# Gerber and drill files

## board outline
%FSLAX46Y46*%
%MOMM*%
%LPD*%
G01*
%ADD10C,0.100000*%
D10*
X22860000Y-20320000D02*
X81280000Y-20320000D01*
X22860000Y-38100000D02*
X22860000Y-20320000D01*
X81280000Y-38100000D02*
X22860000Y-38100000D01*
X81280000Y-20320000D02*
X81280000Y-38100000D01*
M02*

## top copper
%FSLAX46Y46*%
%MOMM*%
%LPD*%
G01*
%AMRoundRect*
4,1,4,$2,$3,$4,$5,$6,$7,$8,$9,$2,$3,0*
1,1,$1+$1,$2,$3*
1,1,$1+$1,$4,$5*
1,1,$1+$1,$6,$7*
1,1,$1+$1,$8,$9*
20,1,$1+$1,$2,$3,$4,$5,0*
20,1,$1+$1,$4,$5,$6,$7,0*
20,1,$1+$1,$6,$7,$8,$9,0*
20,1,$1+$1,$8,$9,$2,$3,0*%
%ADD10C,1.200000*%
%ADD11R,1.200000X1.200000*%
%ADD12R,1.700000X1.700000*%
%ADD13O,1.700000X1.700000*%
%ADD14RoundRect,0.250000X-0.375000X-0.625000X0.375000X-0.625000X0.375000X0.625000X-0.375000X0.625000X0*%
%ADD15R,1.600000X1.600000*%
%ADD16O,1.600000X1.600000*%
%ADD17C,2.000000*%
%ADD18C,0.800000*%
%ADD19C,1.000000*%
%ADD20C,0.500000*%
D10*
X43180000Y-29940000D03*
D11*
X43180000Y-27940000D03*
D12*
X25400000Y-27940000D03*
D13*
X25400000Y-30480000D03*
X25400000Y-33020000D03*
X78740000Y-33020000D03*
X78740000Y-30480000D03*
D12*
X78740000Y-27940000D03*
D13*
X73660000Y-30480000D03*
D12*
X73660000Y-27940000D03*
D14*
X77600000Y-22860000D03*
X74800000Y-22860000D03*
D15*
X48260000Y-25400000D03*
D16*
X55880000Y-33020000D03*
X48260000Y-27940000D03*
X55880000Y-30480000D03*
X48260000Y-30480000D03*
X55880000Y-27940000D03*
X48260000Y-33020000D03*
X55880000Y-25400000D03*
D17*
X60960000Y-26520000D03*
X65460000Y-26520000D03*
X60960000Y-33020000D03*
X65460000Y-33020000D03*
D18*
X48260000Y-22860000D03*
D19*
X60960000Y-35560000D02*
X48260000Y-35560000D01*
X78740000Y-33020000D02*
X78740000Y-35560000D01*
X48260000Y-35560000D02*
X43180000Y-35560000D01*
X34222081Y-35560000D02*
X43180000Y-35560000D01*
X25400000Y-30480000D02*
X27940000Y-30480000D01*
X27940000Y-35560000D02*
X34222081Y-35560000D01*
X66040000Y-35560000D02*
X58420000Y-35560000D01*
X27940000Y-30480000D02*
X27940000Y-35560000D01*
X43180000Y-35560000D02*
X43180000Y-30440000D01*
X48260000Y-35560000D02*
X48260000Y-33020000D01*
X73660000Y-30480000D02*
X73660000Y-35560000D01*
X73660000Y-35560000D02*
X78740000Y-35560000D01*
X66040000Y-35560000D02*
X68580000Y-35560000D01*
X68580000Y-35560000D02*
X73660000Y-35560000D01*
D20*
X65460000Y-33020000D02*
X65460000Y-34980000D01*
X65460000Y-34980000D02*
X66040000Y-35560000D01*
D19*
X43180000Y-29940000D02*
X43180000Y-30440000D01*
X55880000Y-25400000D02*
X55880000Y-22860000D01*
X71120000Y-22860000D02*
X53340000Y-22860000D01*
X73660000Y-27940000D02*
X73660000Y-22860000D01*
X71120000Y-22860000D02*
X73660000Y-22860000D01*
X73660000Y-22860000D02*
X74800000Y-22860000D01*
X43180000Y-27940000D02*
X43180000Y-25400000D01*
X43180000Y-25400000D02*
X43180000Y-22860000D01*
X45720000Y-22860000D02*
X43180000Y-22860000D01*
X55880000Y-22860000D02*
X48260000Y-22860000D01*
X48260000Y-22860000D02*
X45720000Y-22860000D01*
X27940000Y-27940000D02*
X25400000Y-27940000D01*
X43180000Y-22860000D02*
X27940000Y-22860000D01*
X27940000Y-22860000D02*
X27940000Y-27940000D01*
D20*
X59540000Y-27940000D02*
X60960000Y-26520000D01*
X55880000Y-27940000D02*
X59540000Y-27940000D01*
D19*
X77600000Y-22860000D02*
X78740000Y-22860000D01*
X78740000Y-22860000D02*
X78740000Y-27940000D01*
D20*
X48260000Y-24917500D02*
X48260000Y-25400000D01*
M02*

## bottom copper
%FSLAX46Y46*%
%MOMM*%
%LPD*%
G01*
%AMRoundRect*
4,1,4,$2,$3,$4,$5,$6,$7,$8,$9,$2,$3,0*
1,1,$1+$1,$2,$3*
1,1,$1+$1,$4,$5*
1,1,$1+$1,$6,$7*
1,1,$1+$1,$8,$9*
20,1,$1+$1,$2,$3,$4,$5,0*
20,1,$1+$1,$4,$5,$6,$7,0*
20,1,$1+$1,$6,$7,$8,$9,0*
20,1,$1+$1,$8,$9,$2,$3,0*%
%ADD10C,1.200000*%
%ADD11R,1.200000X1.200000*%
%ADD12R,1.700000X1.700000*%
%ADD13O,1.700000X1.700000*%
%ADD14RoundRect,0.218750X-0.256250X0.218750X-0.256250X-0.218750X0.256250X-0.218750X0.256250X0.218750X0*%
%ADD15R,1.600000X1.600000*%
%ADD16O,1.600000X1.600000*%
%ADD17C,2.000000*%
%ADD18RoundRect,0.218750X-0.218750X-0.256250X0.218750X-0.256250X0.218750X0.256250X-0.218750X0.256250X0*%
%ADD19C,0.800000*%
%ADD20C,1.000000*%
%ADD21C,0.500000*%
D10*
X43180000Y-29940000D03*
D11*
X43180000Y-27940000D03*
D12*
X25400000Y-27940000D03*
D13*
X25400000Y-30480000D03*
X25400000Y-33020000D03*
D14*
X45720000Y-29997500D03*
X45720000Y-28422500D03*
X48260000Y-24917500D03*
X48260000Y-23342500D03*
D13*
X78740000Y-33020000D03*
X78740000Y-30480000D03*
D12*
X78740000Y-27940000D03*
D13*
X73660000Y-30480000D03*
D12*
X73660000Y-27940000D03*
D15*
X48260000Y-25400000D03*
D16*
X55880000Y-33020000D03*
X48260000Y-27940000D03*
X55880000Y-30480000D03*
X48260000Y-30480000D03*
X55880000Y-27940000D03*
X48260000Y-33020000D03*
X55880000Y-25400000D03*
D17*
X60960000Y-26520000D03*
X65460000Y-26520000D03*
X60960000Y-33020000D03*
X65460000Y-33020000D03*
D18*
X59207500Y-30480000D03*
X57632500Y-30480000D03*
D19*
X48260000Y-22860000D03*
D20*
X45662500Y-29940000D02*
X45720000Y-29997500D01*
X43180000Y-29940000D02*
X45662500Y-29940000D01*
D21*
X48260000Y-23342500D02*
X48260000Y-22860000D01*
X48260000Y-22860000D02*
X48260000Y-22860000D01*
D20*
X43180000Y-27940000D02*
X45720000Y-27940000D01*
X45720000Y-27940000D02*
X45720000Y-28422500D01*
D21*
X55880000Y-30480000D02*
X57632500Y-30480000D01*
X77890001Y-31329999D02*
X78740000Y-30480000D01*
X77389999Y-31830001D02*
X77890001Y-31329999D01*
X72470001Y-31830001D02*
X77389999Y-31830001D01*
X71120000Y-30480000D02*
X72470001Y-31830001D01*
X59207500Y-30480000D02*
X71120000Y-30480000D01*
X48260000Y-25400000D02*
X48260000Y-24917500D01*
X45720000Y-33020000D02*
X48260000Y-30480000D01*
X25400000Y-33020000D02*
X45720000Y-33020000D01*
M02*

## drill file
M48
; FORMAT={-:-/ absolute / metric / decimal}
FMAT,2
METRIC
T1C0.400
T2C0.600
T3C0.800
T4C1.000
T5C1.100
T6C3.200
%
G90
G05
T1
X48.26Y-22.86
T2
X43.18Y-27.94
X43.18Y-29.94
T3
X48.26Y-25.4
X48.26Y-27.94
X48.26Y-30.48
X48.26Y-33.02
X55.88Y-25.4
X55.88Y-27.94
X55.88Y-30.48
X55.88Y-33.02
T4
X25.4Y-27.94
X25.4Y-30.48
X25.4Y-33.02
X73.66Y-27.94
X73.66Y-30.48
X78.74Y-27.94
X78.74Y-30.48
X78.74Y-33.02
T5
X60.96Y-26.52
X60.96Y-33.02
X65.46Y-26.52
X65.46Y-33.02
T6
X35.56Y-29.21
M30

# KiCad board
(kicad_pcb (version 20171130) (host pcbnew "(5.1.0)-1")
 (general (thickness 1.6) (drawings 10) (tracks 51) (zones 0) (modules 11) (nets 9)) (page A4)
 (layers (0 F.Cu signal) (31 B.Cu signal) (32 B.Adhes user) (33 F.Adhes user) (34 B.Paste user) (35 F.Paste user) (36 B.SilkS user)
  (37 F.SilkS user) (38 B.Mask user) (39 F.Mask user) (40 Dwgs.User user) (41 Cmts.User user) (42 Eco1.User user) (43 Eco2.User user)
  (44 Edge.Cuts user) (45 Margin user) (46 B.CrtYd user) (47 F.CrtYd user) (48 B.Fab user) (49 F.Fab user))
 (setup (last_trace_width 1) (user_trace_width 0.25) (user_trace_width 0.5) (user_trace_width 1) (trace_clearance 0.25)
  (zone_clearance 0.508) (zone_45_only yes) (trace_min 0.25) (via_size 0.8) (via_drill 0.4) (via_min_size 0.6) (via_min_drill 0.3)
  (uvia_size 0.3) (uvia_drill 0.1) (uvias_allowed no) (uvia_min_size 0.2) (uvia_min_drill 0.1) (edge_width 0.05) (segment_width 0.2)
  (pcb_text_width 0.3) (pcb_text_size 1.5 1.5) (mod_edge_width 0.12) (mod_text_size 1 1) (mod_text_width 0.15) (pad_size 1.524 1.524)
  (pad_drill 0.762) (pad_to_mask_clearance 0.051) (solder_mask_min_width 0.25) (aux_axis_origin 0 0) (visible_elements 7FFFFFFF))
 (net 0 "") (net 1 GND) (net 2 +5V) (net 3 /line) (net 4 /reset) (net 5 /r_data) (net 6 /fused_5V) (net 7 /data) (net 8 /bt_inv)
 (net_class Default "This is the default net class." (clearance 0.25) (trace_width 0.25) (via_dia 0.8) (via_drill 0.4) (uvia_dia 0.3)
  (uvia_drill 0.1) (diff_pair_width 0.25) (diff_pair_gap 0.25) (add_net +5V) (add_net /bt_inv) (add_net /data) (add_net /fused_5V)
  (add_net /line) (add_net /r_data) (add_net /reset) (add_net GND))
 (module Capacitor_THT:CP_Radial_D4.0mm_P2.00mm (layer F.Cu) (at 43.18 27.94 270)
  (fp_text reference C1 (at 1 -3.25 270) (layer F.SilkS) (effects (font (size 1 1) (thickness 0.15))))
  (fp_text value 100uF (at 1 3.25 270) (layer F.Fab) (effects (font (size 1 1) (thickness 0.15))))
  (pad 2 thru_hole circle (at 2 0 270) (size 1.2 1.2) (drill 0.6) (layers *.Cu *.Mask) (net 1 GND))
  (pad 1 thru_hole rect (at 0 0 270) (size 1.2 1.2) (drill 0.6) (layers *.Cu *.Mask) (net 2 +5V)))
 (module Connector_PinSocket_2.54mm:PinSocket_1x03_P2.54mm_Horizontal (layer F.Cu) (at 25.4 27.94)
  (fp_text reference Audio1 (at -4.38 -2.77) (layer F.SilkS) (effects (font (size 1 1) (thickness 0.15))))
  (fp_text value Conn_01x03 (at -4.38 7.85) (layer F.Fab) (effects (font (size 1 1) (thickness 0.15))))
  (pad 1 thru_hole rect (at 0 0) (size 1.7 1.7) (drill 1) (layers *.Cu *.Mask) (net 2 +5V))
  (pad 2 thru_hole oval (at 0 2.54) (size 1.7 1.7) (drill 1) (layers *.Cu *.Mask) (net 1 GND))
  (pad 3 thru_hole oval (at 0 5.08) (size 1.7 1.7) (drill 1) (layers *.Cu *.Mask) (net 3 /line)))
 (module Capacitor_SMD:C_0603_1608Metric (layer B.Cu) (at 45.72 29.21 270)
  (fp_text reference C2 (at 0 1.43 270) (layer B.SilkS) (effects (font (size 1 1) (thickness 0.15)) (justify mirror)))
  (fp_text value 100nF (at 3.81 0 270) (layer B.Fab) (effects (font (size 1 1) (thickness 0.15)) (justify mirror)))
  (pad 2 smd roundrect (at 0.7875 0 270) (size 0.875 0.95) (layers B.Cu B.Paste B.Mask) (roundrect_rratio 0.25) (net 1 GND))
  (pad 1 smd roundrect (at -0.7875 0 270) (size 0.875 0.95) (layers B.Cu B.Paste B.Mask) (roundrect_rratio 0.25) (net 2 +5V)))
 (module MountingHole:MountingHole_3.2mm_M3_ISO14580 (layer F.Cu) (at 35.56 29.21)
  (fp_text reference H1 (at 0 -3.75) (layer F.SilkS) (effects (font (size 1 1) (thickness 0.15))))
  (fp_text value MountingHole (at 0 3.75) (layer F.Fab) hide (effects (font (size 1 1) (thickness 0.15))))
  (pad 1 np_thru_hole circle (at 0 0) (size 3.2 3.2) (drill 3.2) (layers *.Cu *.Mask)))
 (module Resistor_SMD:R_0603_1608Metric (layer B.Cu) (at 48.26 24.13 270)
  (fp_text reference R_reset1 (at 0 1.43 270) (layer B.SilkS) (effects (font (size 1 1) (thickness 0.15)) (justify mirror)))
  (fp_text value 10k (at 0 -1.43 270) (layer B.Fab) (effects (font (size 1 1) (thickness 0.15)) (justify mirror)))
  (pad 2 smd roundrect (at 0.7875 0 270) (size 0.875 0.95) (layers B.Cu B.Paste B.Mask) (roundrect_rratio 0.25) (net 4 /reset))
  (pad 1 smd roundrect (at -0.7875 0 270) (size 0.875 0.95) (layers B.Cu B.Paste B.Mask) (roundrect_rratio 0.25) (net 2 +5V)))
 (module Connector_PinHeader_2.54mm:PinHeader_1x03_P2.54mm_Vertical (layer B.Cu) (at 78.74 27.94 180)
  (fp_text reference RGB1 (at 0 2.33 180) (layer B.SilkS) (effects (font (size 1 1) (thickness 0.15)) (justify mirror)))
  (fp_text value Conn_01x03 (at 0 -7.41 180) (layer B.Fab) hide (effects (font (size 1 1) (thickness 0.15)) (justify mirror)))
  (pad 3 thru_hole oval (at 0 -5.08 180) (size 1.7 1.7) (drill 1) (layers *.Cu *.Mask) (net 1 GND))
  (pad 2 thru_hole oval (at 0 -2.54 180) (size 1.7 1.7) (drill 1) (layers *.Cu *.Mask) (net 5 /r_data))
  (pad 1 thru_hole rect (at 0 0 180) (size 1.7 1.7) (drill 1) (layers *.Cu *.Mask) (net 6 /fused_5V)))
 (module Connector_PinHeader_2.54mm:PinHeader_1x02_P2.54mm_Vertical (layer F.Cu) (at 73.66 27.94)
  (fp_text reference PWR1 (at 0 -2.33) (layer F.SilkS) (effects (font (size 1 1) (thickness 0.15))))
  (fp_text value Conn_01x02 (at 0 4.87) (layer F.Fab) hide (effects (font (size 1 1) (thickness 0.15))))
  (pad 2 thru_hole oval (at 0 2.54) (size 1.7 1.7) (drill 1) (layers *.Cu *.Mask) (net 1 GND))
  (pad 1 thru_hole rect (at 0 0) (size 1.7 1.7) (drill 1) (layers *.Cu *.Mask) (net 2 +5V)))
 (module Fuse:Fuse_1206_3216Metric (layer F.Cu) (at 76.2 22.86)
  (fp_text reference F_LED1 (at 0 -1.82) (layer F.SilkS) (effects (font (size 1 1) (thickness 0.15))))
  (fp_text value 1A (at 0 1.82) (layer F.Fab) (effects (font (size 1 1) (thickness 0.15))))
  (pad 2 smd roundrect (at 1.4 0) (size 1.25 1.75) (layers F.Cu F.Paste F.Mask) (roundrect_rratio 0.2) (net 6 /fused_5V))
  (pad 1 smd roundrect (at -1.4 0) (size 1.25 1.75) (layers F.Cu F.Paste F.Mask) (roundrect_rratio 0.2) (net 2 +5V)))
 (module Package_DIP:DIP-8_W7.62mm (layer F.Cu) (at 48.26 25.4)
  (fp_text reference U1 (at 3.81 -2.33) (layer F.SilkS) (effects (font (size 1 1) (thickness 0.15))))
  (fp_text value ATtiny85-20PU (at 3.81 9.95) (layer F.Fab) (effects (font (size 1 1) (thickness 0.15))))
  (pad 1 thru_hole rect (at 0 0) (size 1.6 1.6) (drill 0.8) (layers *.Cu *.Mask) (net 4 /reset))
  (pad 5 thru_hole oval (at 7.62 7.62) (size 1.6 1.6) (drill 0.8) (layers *.Cu *.Mask))
  (pad 2 thru_hole oval (at 0 2.54) (size 1.6 1.6) (drill 0.8) (layers *.Cu *.Mask))
  (pad 6 thru_hole oval (at 7.62 5.08) (size 1.6 1.6) (drill 0.8) (layers *.Cu *.Mask) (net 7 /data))
  (pad 3 thru_hole oval (at 0 5.08) (size 1.6 1.6) (drill 0.8) (layers *.Cu *.Mask) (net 3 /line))
  (pad 7 thru_hole oval (at 7.62 2.54) (size 1.6 1.6) (drill 0.8) (layers *.Cu *.Mask) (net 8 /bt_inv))
  (pad 4 thru_hole oval (at 0 7.62) (size 1.6 1.6) (drill 0.8) (layers *.Cu *.Mask) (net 1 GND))
  (pad 8 thru_hole oval (at 7.62 0) (size 1.6 1.6) (drill 0.8) (layers *.Cu *.Mask) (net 2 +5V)))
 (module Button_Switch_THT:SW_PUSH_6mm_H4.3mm (layer F.Cu) (at 60.96 33.02 90)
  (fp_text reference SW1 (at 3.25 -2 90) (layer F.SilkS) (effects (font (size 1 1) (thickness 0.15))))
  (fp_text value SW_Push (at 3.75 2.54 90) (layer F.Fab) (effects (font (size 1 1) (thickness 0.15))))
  (pad 1 thru_hole circle (at 6.5 0 180) (size 2 2) (drill 1.1) (layers *.Cu *.Mask) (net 8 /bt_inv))
  (pad 2 thru_hole circle (at 6.5 4.5 180) (size 2 2) (drill 1.1) (layers *.Cu *.Mask) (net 1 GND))
  (pad 1 thru_hole circle (at 0 0 180) (size 2 2) (drill 1.1) (layers *.Cu *.Mask) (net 8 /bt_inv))
  (pad 2 thru_hole circle (at 0 4.5 180) (size 2 2) (drill 1.1) (layers *.Cu *.Mask) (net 1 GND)))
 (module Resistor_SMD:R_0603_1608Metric (layer B.Cu) (at 58.42 30.48)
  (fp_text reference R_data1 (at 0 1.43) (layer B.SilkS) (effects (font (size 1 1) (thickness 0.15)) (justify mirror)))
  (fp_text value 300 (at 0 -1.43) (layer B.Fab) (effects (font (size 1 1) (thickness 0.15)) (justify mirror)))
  (pad 2 smd roundrect (at 0.7875 0) (size 0.875 0.95) (layers B.Cu B.Paste B.Mask) (roundrect_rratio 0.25) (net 5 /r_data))
  (pad 1 smd roundrect (at -0.7875 0) (size 0.875 0.95) (layers B.Cu B.Paste B.Mask) (roundrect_rratio 0.25) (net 7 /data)))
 (gr_line (start 22.86 20.32) (end 81.28 20.32) (layer Edge.Cuts) (width 0.1))
 (gr_line (start 22.86 38.1) (end 22.86 20.32) (layer Edge.Cuts) (width 0.1))
 (gr_line (start 81.28 38.1) (end 22.86 38.1) (layer Edge.Cuts) (width 0.1))
 (gr_line (start 81.28 20.32) (end 81.28 38.1) (layer Edge.Cuts) (width 0.1))
 (segment (start 60.96 35.56) (end 48.26 35.56) (width 1) (layer F.Cu) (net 1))
 (segment (start 78.74 33.02) (end 78.74 35.56) (width 1) (layer F.Cu) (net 1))
 (segment (start 48.26 35.56) (end 43.18 35.56) (width 1) (layer F.Cu) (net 1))
 (segment (start 34.222081 35.56) (end 43.18 35.56) (width 1) (layer F.Cu) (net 1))
 (segment (start 25.4 30.48) (end 27.94 30.48) (width 1) (layer F.Cu) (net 1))
 (segment (start 27.94 35.56) (end 34.222081 35.56) (width 1) (layer F.Cu) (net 1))
 (segment (start 66.04 35.56) (end 58.42 35.56) (width 1) (layer F.Cu) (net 1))
 (segment (start 27.94 30.48) (end 27.94 35.56) (width 1) (layer F.Cu) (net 1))
 (segment (start 43.18 35.56) (end 43.18 30.44) (width 1) (layer F.Cu) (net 1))
 (segment (start 48.26 35.56) (end 48.26 33.02) (width 1) (layer F.Cu) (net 1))
 (segment (start 73.66 30.48) (end 73.66 35.56) (width 1) (layer F.Cu) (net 1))
 (segment (start 73.66 35.56) (end 78.74 35.56) (width 1) (layer F.Cu) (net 1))
 (segment (start 66.04 35.56) (end 68.58 35.56) (width 1) (layer F.Cu) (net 1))
 (segment (start 68.58 35.56) (end 73.66 35.56) (width 1) (layer F.Cu) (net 1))
 (segment (start 65.46 33.02) (end 65.46 34.98) (width 0.5) (layer F.Cu) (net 1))
 (segment (start 65.46 34.98) (end 66.04 35.56) (width 0.5) (layer F.Cu) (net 1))
 (segment (start 43.18 29.94) (end 43.18 30.44) (width 1) (layer F.Cu) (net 1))
 (segment (start 45.6625 29.94) (end 45.72 29.9975) (width 1) (layer B.Cu) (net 1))
 (segment (start 43.18 29.94) (end 45.6625 29.94) (width 1) (layer B.Cu) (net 1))
 (segment (start 55.88 25.4) (end 55.88 22.86) (width 1) (layer F.Cu) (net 2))
 (segment (start 71.12 22.86) (end 53.34 22.86) (width 1) (layer F.Cu) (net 2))
 (segment (start 73.66 27.94) (end 73.66 22.86) (width 1) (layer F.Cu) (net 2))
 (segment (start 71.12 22.86) (end 73.66 22.86) (width 1) (layer F.Cu) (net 2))
 (segment (start 73.66 22.86) (end 74.8 22.86) (width 1) (layer F.Cu) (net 2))
 (segment (start 43.18 27.94) (end 43.18 25.4) (width 1) (layer F.Cu) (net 2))
 (segment (start 43.18 25.4) (end 43.18 22.86) (width 1) (layer F.Cu) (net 2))
 (segment (start 45.72 22.86) (end 43.18 22.86) (width 1) (layer F.Cu) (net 2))
 (segment (start 55.88 22.86) (end 48.26 22.86) (width 1) (layer F.Cu) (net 2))
 (segment (start 48.26 22.86) (end 45.72 22.86) (width 1) (layer F.Cu) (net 2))
 (segment (start 27.94 27.94) (end 25.4 27.94) (width 1) (layer F.Cu) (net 2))
 (segment (start 43.18 22.86) (end 27.94 22.86) (width 1) (layer F.Cu) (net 2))
 (segment (start 27.94 22.86) (end 27.94 27.94) (width 1) (layer F.Cu) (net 2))
 (segment (start 48.26 23.3425) (end 48.26 22.86) (width 0.5) (layer B.Cu) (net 2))
 (segment (start 48.26 22.86) (end 48.26 22.86) (width 0.5) (layer B.Cu) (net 2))
 (via (at 48.26 22.86) (size 0.8) (drill 0.4) (layers F.Cu B.Cu) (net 2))
 (segment (start 43.18 27.94) (end 45.72 27.94) (width 1) (layer B.Cu) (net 2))
 (segment (start 45.72 27.94) (end 45.72 28.4225) (width 1) (layer B.Cu) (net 2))
 (segment (start 55.88 30.48) (end 57.6325 30.48) (width 0.5) (layer B.Cu) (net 7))
 (segment (start 59.54 27.94) (end 60.96 26.52) (width 0.5) (layer F.Cu) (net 8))
 (segment (start 55.88 27.94) (end 59.54 27.94) (width 0.5) (layer F.Cu) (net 8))
 (segment (start 77.6 22.86) (end 78.74 22.86) (width 1) (layer F.Cu) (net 6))
 (segment (start 78.74 22.86) (end 78.74 27.94) (width 1) (layer F.Cu) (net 6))
 (segment (start 77.890001 31.329999) (end 78.74 30.48) (width 0.5) (layer B.Cu) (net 5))
 (segment (start 77.389999 31.830001) (end 77.890001 31.329999) (width 0.5) (layer B.Cu) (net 5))
 (segment (start 72.470001 31.830001) (end 77.389999 31.830001) (width 0.5) (layer B.Cu) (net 5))
 (segment (start 71.12 30.48) (end 72.470001 31.830001) (width 0.5) (layer B.Cu) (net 5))
 (segment (start 59.2075 30.48) (end 71.12 30.48) (width 0.5) (layer B.Cu) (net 5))
 (segment (start 48.26 24.9175) (end 48.26 25.4) (width 0.5) (layer F.Cu) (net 4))
 (segment (start 48.26 25.4) (end 48.26 24.9175) (width 0.5) (layer B.Cu) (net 4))
 (segment (start 45.72 33.02) (end 48.26 30.48) (width 0.5) (layer B.Cu) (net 3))
 (segment (start 25.4 33.02) (end 45.72 33.02) (width 0.5) (layer B.Cu) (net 3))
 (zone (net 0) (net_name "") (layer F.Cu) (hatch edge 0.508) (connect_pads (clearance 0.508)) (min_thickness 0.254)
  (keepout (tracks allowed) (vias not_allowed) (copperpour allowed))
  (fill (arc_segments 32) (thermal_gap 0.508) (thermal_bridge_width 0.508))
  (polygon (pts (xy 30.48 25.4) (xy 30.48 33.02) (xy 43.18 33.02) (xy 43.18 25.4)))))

